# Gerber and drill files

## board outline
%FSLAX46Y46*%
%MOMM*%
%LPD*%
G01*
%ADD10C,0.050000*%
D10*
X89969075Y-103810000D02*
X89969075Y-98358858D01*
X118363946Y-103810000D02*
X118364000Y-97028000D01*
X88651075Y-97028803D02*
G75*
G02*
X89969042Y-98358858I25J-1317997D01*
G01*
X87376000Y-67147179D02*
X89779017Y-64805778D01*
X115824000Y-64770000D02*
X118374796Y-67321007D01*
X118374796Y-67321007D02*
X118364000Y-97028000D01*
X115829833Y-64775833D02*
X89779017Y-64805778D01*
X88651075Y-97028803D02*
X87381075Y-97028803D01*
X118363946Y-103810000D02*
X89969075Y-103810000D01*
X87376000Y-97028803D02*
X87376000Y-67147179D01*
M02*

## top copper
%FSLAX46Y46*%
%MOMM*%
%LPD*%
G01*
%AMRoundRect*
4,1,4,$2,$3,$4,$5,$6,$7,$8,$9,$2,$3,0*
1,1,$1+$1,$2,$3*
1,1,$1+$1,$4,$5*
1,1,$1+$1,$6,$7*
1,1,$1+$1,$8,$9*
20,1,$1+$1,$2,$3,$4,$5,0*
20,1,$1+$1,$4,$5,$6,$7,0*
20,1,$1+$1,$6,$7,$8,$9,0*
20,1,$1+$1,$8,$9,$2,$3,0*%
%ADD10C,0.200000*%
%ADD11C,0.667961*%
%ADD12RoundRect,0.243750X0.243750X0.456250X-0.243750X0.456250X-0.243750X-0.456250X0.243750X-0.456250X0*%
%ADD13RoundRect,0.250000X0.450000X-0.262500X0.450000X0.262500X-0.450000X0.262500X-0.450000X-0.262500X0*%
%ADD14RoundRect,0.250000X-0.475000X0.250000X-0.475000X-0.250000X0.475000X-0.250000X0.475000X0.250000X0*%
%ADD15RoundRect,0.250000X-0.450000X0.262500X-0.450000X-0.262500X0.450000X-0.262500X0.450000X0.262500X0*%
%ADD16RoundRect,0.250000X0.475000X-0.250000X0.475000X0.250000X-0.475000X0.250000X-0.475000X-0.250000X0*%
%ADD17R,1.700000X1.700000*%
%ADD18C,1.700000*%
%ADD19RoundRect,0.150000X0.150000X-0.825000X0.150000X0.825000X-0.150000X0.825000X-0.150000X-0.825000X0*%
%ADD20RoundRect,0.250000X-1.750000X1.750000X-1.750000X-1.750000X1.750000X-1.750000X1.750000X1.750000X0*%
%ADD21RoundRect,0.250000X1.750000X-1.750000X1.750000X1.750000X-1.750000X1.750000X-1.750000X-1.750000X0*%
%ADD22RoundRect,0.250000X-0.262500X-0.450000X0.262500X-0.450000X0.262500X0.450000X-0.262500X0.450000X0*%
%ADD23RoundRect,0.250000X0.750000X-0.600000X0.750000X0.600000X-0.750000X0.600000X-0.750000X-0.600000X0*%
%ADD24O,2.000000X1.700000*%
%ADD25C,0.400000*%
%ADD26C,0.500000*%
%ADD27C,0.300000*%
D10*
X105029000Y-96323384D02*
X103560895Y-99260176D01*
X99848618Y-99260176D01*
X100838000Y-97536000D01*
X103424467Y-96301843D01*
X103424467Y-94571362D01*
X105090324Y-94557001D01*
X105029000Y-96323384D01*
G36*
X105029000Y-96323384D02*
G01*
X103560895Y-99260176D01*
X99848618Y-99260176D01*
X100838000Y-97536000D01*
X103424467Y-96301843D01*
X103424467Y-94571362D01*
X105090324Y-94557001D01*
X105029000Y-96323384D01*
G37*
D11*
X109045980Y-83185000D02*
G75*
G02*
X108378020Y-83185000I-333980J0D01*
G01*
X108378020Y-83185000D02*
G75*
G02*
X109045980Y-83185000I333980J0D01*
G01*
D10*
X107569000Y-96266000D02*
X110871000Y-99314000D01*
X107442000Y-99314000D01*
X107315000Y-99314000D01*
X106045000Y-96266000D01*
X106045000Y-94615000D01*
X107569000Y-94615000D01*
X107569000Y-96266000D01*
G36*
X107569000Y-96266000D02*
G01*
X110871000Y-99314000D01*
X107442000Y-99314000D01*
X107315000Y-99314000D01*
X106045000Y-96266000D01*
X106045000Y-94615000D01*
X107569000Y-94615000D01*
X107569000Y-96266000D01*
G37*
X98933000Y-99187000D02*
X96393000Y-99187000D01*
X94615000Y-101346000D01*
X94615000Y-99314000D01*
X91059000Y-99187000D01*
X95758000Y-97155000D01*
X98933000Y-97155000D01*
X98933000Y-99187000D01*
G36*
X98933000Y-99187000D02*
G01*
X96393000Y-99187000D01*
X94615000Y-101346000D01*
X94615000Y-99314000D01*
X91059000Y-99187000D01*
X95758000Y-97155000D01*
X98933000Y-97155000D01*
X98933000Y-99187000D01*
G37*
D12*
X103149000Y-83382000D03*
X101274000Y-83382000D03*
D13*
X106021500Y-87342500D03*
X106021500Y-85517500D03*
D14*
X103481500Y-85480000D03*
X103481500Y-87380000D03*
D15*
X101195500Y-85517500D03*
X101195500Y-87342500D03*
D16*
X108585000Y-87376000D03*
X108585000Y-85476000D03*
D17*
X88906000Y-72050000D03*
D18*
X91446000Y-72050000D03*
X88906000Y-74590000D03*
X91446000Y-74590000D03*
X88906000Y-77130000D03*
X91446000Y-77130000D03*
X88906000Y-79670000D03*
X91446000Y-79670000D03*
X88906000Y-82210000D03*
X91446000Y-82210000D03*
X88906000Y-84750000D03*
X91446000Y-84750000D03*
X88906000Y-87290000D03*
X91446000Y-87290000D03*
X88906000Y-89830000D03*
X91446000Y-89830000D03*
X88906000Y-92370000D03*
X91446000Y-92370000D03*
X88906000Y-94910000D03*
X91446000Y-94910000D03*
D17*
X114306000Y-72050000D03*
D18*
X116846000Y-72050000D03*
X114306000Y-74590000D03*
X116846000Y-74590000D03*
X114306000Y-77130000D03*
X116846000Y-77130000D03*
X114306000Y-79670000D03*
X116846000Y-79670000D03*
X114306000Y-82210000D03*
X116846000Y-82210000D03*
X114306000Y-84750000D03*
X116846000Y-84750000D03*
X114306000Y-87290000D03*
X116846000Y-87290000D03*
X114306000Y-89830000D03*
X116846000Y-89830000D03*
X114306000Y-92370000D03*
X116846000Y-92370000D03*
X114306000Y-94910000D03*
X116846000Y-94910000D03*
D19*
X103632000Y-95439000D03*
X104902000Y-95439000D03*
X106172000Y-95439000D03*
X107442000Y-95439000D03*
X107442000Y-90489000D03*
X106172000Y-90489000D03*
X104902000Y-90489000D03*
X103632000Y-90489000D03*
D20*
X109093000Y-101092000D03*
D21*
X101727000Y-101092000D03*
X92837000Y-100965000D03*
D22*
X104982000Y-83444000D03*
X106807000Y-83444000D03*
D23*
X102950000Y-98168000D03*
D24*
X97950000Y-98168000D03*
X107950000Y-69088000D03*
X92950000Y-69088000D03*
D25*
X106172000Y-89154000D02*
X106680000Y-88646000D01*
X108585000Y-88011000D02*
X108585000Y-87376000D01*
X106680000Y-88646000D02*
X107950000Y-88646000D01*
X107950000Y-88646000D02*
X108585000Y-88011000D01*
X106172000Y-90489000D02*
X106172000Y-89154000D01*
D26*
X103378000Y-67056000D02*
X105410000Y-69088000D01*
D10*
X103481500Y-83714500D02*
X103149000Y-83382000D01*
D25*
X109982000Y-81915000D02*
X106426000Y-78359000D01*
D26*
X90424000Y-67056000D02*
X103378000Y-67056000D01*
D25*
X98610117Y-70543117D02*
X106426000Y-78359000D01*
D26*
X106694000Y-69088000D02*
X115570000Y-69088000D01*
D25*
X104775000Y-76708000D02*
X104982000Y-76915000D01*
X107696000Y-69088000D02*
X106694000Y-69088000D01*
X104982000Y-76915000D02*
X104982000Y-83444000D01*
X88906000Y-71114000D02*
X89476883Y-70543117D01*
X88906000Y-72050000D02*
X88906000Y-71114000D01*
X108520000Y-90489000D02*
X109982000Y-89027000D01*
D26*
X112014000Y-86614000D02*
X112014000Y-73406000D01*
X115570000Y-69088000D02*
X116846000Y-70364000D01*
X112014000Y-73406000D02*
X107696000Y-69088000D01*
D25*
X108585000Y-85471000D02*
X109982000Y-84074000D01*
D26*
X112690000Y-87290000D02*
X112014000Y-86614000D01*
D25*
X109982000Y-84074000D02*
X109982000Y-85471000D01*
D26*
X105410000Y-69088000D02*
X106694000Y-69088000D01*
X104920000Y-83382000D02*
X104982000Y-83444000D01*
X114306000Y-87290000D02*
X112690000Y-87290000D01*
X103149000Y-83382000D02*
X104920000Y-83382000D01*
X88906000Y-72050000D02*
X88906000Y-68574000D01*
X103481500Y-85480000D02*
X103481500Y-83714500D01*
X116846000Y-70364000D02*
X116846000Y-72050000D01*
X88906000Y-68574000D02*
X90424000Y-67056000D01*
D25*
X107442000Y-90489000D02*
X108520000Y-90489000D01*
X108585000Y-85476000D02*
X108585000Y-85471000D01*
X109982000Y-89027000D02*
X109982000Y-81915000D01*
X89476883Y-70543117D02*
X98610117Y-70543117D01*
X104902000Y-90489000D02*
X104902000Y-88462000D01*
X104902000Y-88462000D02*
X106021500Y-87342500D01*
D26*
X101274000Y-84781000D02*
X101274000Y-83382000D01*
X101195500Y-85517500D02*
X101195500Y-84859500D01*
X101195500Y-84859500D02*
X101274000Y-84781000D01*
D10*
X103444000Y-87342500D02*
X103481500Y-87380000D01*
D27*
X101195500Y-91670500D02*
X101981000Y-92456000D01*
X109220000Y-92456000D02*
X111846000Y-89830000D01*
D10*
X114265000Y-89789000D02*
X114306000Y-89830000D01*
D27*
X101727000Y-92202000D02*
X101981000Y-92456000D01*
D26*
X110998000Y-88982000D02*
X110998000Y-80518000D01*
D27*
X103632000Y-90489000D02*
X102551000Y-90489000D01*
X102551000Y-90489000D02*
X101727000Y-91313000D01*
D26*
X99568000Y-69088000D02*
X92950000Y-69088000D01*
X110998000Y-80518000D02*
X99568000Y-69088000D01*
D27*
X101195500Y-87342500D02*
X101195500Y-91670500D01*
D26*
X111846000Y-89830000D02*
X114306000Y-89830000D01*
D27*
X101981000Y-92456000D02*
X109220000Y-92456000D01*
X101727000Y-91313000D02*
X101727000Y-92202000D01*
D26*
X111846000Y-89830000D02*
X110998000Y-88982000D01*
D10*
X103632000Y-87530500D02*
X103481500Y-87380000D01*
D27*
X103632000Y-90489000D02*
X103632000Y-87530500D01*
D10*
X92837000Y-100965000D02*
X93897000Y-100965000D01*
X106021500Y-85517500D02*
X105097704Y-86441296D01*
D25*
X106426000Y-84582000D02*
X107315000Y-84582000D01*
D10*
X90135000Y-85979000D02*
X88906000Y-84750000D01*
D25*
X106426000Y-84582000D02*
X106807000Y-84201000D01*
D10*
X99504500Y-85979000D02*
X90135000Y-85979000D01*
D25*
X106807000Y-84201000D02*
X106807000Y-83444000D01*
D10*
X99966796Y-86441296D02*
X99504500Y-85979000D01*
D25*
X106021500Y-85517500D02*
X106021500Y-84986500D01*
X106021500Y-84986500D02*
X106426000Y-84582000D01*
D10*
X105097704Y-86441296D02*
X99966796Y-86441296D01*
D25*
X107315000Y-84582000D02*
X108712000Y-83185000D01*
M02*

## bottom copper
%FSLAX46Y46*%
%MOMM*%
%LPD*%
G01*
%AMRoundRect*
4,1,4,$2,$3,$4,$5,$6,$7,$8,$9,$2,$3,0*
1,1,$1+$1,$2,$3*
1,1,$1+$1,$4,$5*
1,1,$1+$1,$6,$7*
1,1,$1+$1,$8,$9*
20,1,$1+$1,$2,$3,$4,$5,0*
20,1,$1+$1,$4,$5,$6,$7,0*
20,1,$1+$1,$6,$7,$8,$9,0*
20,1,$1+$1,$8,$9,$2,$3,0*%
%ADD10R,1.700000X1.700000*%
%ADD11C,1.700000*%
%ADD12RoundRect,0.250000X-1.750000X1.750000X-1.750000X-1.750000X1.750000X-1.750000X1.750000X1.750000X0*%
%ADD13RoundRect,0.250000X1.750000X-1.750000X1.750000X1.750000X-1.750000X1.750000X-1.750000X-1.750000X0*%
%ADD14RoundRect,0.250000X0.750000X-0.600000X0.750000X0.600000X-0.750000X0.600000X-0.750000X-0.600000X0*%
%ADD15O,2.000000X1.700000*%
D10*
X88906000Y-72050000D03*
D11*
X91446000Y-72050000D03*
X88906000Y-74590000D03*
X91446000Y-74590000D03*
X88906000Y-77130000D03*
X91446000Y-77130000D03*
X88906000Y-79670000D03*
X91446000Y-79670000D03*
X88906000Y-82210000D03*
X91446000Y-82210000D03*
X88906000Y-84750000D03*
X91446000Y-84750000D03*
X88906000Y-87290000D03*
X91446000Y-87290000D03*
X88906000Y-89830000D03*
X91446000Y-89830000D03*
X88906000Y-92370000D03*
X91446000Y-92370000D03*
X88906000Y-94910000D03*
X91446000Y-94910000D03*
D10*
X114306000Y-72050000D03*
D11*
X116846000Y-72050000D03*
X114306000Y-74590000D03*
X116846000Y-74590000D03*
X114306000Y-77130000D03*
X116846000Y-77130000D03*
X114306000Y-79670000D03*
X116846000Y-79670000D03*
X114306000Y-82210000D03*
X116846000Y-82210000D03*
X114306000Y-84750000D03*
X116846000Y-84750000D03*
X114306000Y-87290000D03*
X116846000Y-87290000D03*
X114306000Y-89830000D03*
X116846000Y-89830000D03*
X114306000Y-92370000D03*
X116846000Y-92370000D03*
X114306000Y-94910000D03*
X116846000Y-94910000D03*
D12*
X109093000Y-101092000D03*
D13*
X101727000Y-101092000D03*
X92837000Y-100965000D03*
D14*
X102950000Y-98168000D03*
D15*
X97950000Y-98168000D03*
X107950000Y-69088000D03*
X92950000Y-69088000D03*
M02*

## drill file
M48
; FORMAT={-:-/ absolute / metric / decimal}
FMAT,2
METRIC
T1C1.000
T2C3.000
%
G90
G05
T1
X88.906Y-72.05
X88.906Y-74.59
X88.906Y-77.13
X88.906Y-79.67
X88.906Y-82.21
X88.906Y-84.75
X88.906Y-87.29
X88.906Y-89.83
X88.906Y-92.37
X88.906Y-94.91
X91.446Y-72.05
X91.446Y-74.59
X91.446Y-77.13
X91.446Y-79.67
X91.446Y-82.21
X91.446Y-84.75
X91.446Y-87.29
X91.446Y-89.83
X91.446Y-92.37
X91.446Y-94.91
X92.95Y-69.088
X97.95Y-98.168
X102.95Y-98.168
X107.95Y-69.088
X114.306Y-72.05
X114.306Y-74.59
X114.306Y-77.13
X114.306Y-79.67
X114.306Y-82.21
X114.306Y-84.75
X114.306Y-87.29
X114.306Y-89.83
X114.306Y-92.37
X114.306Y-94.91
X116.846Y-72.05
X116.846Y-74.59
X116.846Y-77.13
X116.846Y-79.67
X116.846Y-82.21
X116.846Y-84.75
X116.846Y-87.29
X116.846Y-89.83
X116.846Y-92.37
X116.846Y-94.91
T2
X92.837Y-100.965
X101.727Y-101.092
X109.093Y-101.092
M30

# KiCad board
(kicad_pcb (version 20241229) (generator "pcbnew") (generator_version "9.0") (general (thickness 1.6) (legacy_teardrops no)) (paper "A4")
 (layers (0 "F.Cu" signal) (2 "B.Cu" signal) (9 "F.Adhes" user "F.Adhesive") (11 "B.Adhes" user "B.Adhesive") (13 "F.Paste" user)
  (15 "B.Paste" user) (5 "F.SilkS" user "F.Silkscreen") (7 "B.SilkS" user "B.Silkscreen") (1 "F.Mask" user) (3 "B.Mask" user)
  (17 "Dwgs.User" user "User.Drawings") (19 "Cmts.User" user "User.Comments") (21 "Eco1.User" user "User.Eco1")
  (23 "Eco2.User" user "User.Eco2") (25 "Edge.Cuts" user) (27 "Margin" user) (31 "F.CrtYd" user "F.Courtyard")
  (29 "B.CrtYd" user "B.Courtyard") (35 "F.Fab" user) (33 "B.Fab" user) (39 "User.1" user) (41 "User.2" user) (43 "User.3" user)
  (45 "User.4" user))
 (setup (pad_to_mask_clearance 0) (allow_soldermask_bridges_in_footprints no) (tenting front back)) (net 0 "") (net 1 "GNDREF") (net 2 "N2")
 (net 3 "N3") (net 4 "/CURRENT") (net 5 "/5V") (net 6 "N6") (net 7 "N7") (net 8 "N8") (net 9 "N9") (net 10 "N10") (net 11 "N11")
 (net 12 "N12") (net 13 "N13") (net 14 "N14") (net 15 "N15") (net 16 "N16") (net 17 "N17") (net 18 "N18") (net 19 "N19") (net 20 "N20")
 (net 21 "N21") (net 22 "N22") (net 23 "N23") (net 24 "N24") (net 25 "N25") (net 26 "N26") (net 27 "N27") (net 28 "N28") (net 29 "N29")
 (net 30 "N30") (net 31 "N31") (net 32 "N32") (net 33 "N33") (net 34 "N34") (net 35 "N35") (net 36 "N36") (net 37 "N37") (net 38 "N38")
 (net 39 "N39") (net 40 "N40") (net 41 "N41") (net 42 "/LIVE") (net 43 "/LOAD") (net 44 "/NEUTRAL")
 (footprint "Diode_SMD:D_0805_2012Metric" (layer "F.Cu") (at 102.2115 83.382 180)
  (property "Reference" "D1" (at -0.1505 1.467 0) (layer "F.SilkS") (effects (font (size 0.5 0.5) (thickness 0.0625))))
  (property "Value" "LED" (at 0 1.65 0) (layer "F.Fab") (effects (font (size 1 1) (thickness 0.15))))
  (pad "1" smd roundrect (at -0.9375 0 180) (size 0.975 1.4) (layers "F.Cu" "F.Mask" "F.Paste") (roundrect_rratio 0.25) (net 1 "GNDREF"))
  (pad "2" smd roundrect (at 0.9375 0 180) (size 0.975 1.4) (layers "F.Cu" "F.Mask" "F.Paste") (roundrect_rratio 0.25) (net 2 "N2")))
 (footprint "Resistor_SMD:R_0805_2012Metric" (layer "F.Cu") (at 106.0215 86.43 90)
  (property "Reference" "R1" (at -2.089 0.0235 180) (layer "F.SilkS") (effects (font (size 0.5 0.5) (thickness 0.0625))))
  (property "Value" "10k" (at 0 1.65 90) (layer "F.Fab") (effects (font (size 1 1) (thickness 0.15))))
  (pad "1" smd roundrect (at -0.9125 0 90) (size 1.025 1.4) (layers "F.Cu" "F.Mask" "F.Paste") (roundrect_rratio 0.243902) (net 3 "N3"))
  (pad "2" smd roundrect (at 0.9125 0 90) (size 1.025 1.4) (layers "F.Cu" "F.Mask" "F.Paste") (roundrect_rratio 0.243902) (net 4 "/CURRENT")))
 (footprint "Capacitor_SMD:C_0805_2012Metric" (layer "F.Cu") (at 103.4815 86.43 -90)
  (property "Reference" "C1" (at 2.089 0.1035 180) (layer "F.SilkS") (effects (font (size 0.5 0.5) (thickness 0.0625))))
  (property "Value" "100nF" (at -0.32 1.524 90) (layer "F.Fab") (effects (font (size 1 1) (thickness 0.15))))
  (pad "1" smd roundrect (at -0.95 0 270) (size 1 1.45) (layers "F.Cu" "F.Mask" "F.Paste") (roundrect_rratio 0.25) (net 1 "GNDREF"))
  (pad "2" smd roundrect (at 0.95 0 270) (size 1 1.45) (layers "F.Cu" "F.Mask" "F.Paste") (roundrect_rratio 0.25) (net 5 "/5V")))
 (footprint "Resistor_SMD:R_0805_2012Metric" (layer "F.Cu") (at 101.1955 86.43 -90)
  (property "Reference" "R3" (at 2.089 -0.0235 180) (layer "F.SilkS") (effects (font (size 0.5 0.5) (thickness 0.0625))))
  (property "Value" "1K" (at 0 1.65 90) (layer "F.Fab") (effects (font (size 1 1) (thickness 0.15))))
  (pad "1" smd roundrect (at -0.9125 0 270) (size 1.025 1.4) (layers "F.Cu" "F.Mask" "F.Paste") (roundrect_rratio 0.243902) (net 2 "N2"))
  (pad "2" smd roundrect (at 0.9125 0 270) (size 1.025 1.4) (layers "F.Cu" "F.Mask" "F.Paste") (roundrect_rratio 0.243902) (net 5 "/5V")))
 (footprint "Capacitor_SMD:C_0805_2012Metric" (layer "F.Cu") (at 108.585 86.426 90)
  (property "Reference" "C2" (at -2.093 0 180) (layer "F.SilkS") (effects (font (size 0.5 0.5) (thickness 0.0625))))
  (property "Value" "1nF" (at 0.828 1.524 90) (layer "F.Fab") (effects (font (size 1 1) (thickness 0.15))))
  (pad "1" smd roundrect (at -0.95 0 90) (size 1 1.45) (layers "F.Cu" "F.Mask" "F.Paste") (roundrect_rratio 0.25) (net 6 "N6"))
  (pad "2" smd roundrect (at 0.95 0 90) (size 1 1.45) (layers "F.Cu" "F.Mask" "F.Paste") (roundrect_rratio 0.25) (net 1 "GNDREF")))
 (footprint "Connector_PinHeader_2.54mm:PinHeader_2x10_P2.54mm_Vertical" (layer "F.Cu") (at 88.906 72.05)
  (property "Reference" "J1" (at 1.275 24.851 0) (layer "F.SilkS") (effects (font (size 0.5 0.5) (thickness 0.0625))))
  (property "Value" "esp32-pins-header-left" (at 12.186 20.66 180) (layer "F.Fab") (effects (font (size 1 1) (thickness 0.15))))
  (pad "1" thru_hole rect (at 0 0) (size 1.7 1.7) (drill 1) (layers "*.Cu" "*.Mask") (remove_unused_layers no) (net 1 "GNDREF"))
  (pad "2" thru_hole circle (at 2.54 0) (size 1.7 1.7) (drill 1) (layers "*.Cu" "*.Mask") (remove_unused_layers no) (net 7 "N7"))
  (pad "3" thru_hole circle (at 0 2.54) (size 1.7 1.7) (drill 1) (layers "*.Cu" "*.Mask") (remove_unused_layers no) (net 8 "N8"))
  (pad "4" thru_hole circle (at 2.54 2.54) (size 1.7 1.7) (drill 1) (layers "*.Cu" "*.Mask") (remove_unused_layers no) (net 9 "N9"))
  (pad "5" thru_hole circle (at 0 5.08) (size 1.7 1.7) (drill 1) (layers "*.Cu" "*.Mask") (remove_unused_layers no) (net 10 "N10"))
  (pad "6" thru_hole circle (at 2.54 5.08) (size 1.7 1.7) (drill 1) (layers "*.Cu" "*.Mask") (remove_unused_layers no) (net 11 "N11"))
  (pad "7" thru_hole circle (at 0 7.62) (size 1.7 1.7) (drill 1) (layers "*.Cu" "*.Mask") (remove_unused_layers no) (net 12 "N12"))
  (pad "8" thru_hole circle (at 2.54 7.62) (size 1.7 1.7) (drill 1) (layers "*.Cu" "*.Mask") (remove_unused_layers no) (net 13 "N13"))
  (pad "9" thru_hole circle (at 0 10.16) (size 1.7 1.7) (drill 1) (layers "*.Cu" "*.Mask") (remove_unused_layers no) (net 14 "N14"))
  (pad "10" thru_hole circle (at 2.54 10.16) (size 1.7 1.7) (drill 1) (layers "*.Cu" "*.Mask") (remove_unused_layers no) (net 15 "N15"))
  (pad "11" thru_hole circle (at 0 12.7) (size 1.7 1.7) (drill 1) (layers "*.Cu" "*.Mask") (remove_unused_layers no) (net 4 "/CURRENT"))
  (pad "12" thru_hole circle (at 2.54 12.7) (size 1.7 1.7) (drill 1) (layers "*.Cu" "*.Mask") (remove_unused_layers no) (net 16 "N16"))
  (pad "13" thru_hole circle (at 0 15.24) (size 1.7 1.7) (drill 1) (layers "*.Cu" "*.Mask") (remove_unused_layers no) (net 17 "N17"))
  (pad "14" thru_hole circle (at 2.54 15.24) (size 1.7 1.7) (drill 1) (layers "*.Cu" "*.Mask") (remove_unused_layers no) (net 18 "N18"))
  (pad "15" thru_hole circle (at 0 17.78) (size 1.7 1.7) (drill 1) (layers "*.Cu" "*.Mask") (remove_unused_layers no) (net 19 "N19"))
  (pad "16" thru_hole circle (at 2.54 17.78) (size 1.7 1.7) (drill 1) (layers "*.Cu" "*.Mask") (remove_unused_layers no) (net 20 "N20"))
  (pad "17" thru_hole circle (at 0 20.32) (size 1.7 1.7) (drill 1) (layers "*.Cu" "*.Mask") (remove_unused_layers no) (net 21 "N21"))
  (pad "18" thru_hole circle (at 2.54 20.32) (size 1.7 1.7) (drill 1) (layers "*.Cu" "*.Mask") (remove_unused_layers no) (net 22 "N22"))
  (pad "19" thru_hole circle (at 0 22.86) (size 1.7 1.7) (drill 1) (layers "*.Cu" "*.Mask") (remove_unused_layers no) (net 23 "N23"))
  (pad "20" thru_hole circle (at 2.54 22.86) (size 1.7 1.7) (drill 1) (layers "*.Cu" "*.Mask") (remove_unused_layers no) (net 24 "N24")))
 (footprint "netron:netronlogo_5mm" (layer "F.Cu") (at 95.25 74.041)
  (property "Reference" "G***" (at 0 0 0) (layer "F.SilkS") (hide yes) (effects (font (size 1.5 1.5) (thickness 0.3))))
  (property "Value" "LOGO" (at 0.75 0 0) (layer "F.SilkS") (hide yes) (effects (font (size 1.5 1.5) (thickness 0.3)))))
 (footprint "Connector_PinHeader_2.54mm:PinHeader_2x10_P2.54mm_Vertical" (layer "F.Cu") (at 114.306 72.05)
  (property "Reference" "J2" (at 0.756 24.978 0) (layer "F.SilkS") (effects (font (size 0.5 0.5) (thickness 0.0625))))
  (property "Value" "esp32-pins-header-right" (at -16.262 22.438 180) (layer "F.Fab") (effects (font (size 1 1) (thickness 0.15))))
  (pad "1" thru_hole rect (at 0 0) (size 1.7 1.7) (drill 1) (layers "*.Cu" "*.Mask") (remove_unused_layers no) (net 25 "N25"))
  (pad "2" thru_hole circle (at 2.54 0) (size 1.7 1.7) (drill 1) (layers "*.Cu" "*.Mask") (remove_unused_layers no) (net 1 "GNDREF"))
  (pad "3" thru_hole circle (at 0 2.54) (size 1.7 1.7) (drill 1) (layers "*.Cu" "*.Mask") (remove_unused_layers no) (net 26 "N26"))
  (pad "4" thru_hole circle (at 2.54 2.54) (size 1.7 1.7) (drill 1) (layers "*.Cu" "*.Mask") (remove_unused_layers no) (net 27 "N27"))
  (pad "5" thru_hole circle (at 0 5.08) (size 1.7 1.7) (drill 1) (layers "*.Cu" "*.Mask") (remove_unused_layers no) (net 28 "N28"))
  (pad "6" thru_hole circle (at 2.54 5.08) (size 1.7 1.7) (drill 1) (layers "*.Cu" "*.Mask") (remove_unused_layers no) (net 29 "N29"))
  (pad "7" thru_hole circle (at 0 7.62) (size 1.7 1.7) (drill 1) (layers "*.Cu" "*.Mask") (remove_unused_layers no) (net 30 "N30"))
  (pad "8" thru_hole circle (at 2.54 7.62) (size 1.7 1.7) (drill 1) (layers "*.Cu" "*.Mask") (remove_unused_layers no) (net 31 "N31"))
  (pad "9" thru_hole circle (at 0 10.16) (size 1.7 1.7) (drill 1) (layers "*.Cu" "*.Mask") (remove_unused_layers no) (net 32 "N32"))
  (pad "10" thru_hole circle (at 2.54 10.16) (size 1.7 1.7) (drill 1) (layers "*.Cu" "*.Mask") (remove_unused_layers no) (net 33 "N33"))
  (pad "11" thru_hole circle (at 0 12.7) (size 1.7 1.7) (drill 1) (layers "*.Cu" "*.Mask") (remove_unused_layers no) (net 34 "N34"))
  (pad "12" thru_hole circle (at 2.54 12.7) (size 1.7 1.7) (drill 1) (layers "*.Cu" "*.Mask") (remove_unused_layers no) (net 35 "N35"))
  (pad "13" thru_hole circle (at 0 15.24) (size 1.7 1.7) (drill 1) (layers "*.Cu" "*.Mask") (remove_unused_layers no) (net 1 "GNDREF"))
  (pad "14" thru_hole circle (at 2.54 15.24) (size 1.7 1.7) (drill 1) (layers "*.Cu" "*.Mask") (remove_unused_layers no) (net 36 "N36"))
  (pad "15" thru_hole circle (at 0 17.78) (size 1.7 1.7) (drill 1) (layers "*.Cu" "*.Mask") (remove_unused_layers no) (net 5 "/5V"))
  (pad "16" thru_hole circle (at 2.54 17.78) (size 1.7 1.7) (drill 1) (layers "*.Cu" "*.Mask") (remove_unused_layers no) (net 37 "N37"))
  (pad "17" thru_hole circle (at 0 20.32) (size 1.7 1.7) (drill 1) (layers "*.Cu" "*.Mask") (remove_unused_layers no) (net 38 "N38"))
  (pad "18" thru_hole circle (at 2.54 20.32) (size 1.7 1.7) (drill 1) (layers "*.Cu" "*.Mask") (remove_unused_layers no) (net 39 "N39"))
  (pad "19" thru_hole circle (at 0 22.86) (size 1.7 1.7) (drill 1) (layers "*.Cu" "*.Mask") (remove_unused_layers no) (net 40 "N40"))
  (pad "20" thru_hole circle (at 2.54 22.86) (size 1.7 1.7) (drill 1) (layers "*.Cu" "*.Mask") (remove_unused_layers no) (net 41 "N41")))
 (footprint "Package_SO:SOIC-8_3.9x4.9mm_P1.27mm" (layer "F.Cu") (at 105.537 92.964 90)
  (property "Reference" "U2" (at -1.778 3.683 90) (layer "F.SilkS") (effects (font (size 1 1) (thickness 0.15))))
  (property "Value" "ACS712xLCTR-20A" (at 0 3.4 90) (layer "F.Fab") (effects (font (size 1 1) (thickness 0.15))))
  (pad "1" smd roundrect (at -2.475 -1.905 90) (size 1.95 0.6) (layers "F.Cu" "F.Mask" "F.Paste") (roundrect_rratio 0.25) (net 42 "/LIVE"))
  (pad "2" smd roundrect (at -2.475 -0.635 90) (size 1.95 0.6) (layers "F.Cu" "F.Mask" "F.Paste") (roundrect_rratio 0.25) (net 42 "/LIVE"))
  (pad "3" smd roundrect (at -2.475 0.635 90) (size 1.95 0.6) (layers "F.Cu" "F.Mask" "F.Paste") (roundrect_rratio 0.25) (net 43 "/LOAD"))
  (pad "4" smd roundrect (at -2.475 1.905 90) (size 1.95 0.6) (layers "F.Cu" "F.Mask" "F.Paste") (roundrect_rratio 0.25) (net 43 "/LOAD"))
  (pad "5" smd roundrect (at 2.475 1.905 90) (size 1.95 0.6) (layers "F.Cu" "F.Mask" "F.Paste") (roundrect_rratio 0.25) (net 1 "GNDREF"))
  (pad "6" smd roundrect (at 2.475 0.635 90) (size 1.95 0.6) (layers "F.Cu" "F.Mask" "F.Paste") (roundrect_rratio 0.25) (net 6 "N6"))
  (pad "7" smd roundrect (at 2.475 -0.635 90) (size 1.95 0.6) (layers "F.Cu" "F.Mask" "F.Paste") (roundrect_rratio 0.25) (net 3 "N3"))
  (pad "8" smd roundrect (at 2.475 -1.905 90) (size 1.95 0.6) (layers "F.Cu" "F.Mask" "F.Paste") (roundrect_rratio 0.25) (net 5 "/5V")))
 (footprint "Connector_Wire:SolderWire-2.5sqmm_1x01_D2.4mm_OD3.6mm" (layer "F.Cu") (at 109.093 101.092 -90)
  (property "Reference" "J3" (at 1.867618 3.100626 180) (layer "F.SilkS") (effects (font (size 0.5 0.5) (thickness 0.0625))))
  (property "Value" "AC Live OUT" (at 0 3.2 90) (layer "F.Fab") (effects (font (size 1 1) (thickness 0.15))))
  (pad "1" thru_hole roundrect (at 0 0 270) (size 4 4) (drill 3) (layers "*.Cu" "*.Mask") (remove_unused_layers no)
   (roundrect_rratio 0.0625) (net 43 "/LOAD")))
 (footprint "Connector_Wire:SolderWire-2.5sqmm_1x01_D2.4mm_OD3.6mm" (layer "F.Cu") (at 101.727 101.092 90)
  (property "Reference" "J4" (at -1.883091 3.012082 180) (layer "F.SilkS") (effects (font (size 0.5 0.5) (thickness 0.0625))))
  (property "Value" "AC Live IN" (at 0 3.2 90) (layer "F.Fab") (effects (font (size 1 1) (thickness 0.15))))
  (pad "1" thru_hole roundrect (at 0 0 90) (size 4 4) (drill 3) (layers "*.Cu" "*.Mask") (remove_unused_layers no) (roundrect_rratio 0.0625)
   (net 42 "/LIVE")))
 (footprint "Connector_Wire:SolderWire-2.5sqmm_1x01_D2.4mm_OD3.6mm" (layer "F.Cu") (at 92.837 100.965 90)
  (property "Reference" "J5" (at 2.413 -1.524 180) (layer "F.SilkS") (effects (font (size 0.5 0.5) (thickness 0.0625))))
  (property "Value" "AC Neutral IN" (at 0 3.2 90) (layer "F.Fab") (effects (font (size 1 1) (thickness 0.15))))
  (pad "1" thru_hole roundrect (at 0 0 90) (size 4 4) (drill 3) (layers "*.Cu" "*.Mask") (remove_unused_layers no) (roundrect_rratio 0.0625)
   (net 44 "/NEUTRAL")))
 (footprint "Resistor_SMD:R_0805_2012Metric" (layer "F.Cu") (at 105.8945 83.444)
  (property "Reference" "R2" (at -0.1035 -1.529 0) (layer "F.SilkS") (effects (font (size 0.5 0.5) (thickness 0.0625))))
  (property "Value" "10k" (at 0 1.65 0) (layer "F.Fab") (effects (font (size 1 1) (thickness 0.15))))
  (pad "1" smd roundrect (at -0.9125 0) (size 1.025 1.4) (layers "F.Cu" "F.Mask" "F.Paste") (roundrect_rratio 0.243902) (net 1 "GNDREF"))
  (pad "2" smd roundrect (at 0.9125 0) (size 1.025 1.4) (layers "F.Cu" "F.Mask" "F.Paste") (roundrect_rratio 0.243902) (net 4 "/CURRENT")))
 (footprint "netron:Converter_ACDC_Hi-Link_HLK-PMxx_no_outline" (layer "B.Cu") (at 102.95 98.168 90)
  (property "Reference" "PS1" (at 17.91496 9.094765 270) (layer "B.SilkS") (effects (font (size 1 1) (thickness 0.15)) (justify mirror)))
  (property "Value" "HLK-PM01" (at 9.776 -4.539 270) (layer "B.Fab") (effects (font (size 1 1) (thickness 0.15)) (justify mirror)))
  (pad "1" thru_hole roundrect (at 0 0 90) (size 1.7 2) (drill 1) (layers "*.Cu" "*.Mask") (remove_unused_layers no)
   (roundrect_rratio 0.147059) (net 42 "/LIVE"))
  (pad "2" thru_hole oval (at 0 -5 90) (size 1.7 2) (drill 1) (layers "*.Cu" "*.Mask") (remove_unused_layers no) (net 44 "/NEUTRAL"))
  (pad "3" thru_hole oval (at 29.08 5 90) (size 1.7 2) (drill 1) (layers "*.Cu" "*.Mask") (remove_unused_layers no) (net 1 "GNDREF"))
  (pad "4" thru_hole oval (at 29.08 -10 90) (size 1.7 2) (drill 1) (layers "*.Cu" "*.Mask") (remove_unused_layers no) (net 5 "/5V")))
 (gr_poly
  (pts (xy 100.838 97.536) (xy 103.424467 96.301843) (xy 103.424467 94.571362) (xy 105.090324 94.557001) (xy 105.029 96.323384)
   (xy 103.560895 99.260176) (xy 99.848618 99.260176))
  (stroke (width 0.2) (type solid)) (fill yes) (layer "F.Cu") (net 42))
 (gr_circle (center 108.712 83.185) (end 109.22 83.439) (stroke (width 0.2) (type solid)) (fill yes) (layer "F.Cu") (net 4))
 (gr_poly
  (pts (xy 107.569 94.615) (xy 106.045 94.615) (xy 106.045 96.266) (xy 107.315 99.314) (xy 107.442 99.314) (xy 110.871 99.314)
   (xy 107.569 96.266))
  (stroke (width 0.2) (type solid)) (fill yes) (layer "F.Cu") (net 43))
 (gr_poly
  (pts (xy 91.059 99.187) (xy 95.758 97.155) (xy 98.933 97.155) (xy 98.933 99.187) (xy 96.393 99.187) (xy 94.615 101.346) (xy 94.615 99.314))
  (stroke (width 0.2) (type solid)) (fill yes) (layer "F.Cu") (net 44))
 (gr_line (start 89.969075 103.81) (end 89.969075 98.358858) (stroke (width 0.05) (type default)) (layer "Edge.Cuts"))
 (gr_line (start 118.363946 103.81) (end 118.364 97.028) (stroke (width 0.05) (type default)) (layer "Edge.Cuts"))
 (gr_arc (start 88.651075 97.028803) (mid 89.58733 97.419102) (end 89.969075 98.358858) (stroke (width 0.05) (type default))
  (layer "Edge.Cuts"))
 (gr_line (start 87.376 67.147179) (end 89.779017 64.805778) (stroke (width 0.05) (type default)) (layer "Edge.Cuts"))
 (gr_line (start 115.824 64.77) (end 118.374796 67.321007) (stroke (width 0.05) (type default)) (layer "Edge.Cuts"))
 (gr_line (start 118.374796 67.321007) (end 118.364 97.028) (stroke (width 0.05) (type default)) (layer "Edge.Cuts"))
 (gr_line (start 115.829833 64.775833) (end 89.779017 64.805778) (stroke (width 0.05) (type default)) (layer "Edge.Cuts"))
 (gr_line (start 88.651075 97.028803) (end 87.381075 97.028803) (stroke (width 0.05) (type default)) (layer "Edge.Cuts"))
 (gr_line (start 118.363946 103.81) (end 89.969075 103.81) (stroke (width 0.05) (type default)) (layer "Edge.Cuts"))
 (gr_line (start 87.376 97.028803) (end 87.376 67.147179) (stroke (width 0.05) (type default)) (layer "Edge.Cuts"))
 (segment (start 106.172 89.154) (end 106.68 88.646) (width 0.4) (layer "F.Cu") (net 6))
 (segment (start 108.585 88.011) (end 108.585 87.376) (width 0.4) (layer "F.Cu") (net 6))
 (segment (start 106.68 88.646) (end 107.95 88.646) (width 0.4) (layer "F.Cu") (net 6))
 (segment (start 107.95 88.646) (end 108.585 88.011) (width 0.4) (layer "F.Cu") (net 6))
 (segment (start 106.172 90.489) (end 106.172 89.154) (width 0.4) (layer "F.Cu") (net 6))
 (segment (start 103.378 67.056) (end 105.41 69.088) (width 0.5) (layer "F.Cu") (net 1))
 (segment (start 103.4815 83.7145) (end 103.149 83.382) (width 0.2) (layer "F.Cu") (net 1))
 (segment (start 109.982 81.915) (end 106.426 78.359) (width 0.4) (layer "F.Cu") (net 1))
 (segment (start 90.424 67.056) (end 103.378 67.056) (width 0.5) (layer "F.Cu") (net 1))
 (segment (start 98.610117 70.543117) (end 106.426 78.359) (width 0.4) (layer "F.Cu") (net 1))
 (segment (start 106.694 69.088) (end 115.57 69.088) (width 0.5) (layer "F.Cu") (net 1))
 (segment (start 104.775 76.708) (end 104.982 76.915) (width 0.4) (layer "F.Cu") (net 1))
 (segment (start 107.696 69.088) (end 106.694 69.088) (width 0.4) (layer "F.Cu") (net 1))
 (segment (start 104.982 76.915) (end 104.982 83.444) (width 0.4) (layer "F.Cu") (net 1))
 (segment (start 88.906 71.114) (end 89.476883 70.543117) (width 0.4) (layer "F.Cu") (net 1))
 (segment (start 88.906 72.05) (end 88.906 71.114) (width 0.4) (layer "F.Cu") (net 1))
 (segment (start 108.52 90.489) (end 109.982 89.027) (width 0.4) (layer "F.Cu") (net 1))
 (segment (start 112.014 86.614) (end 112.014 73.406) (width 0.5) (layer "F.Cu") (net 1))
 (segment (start 115.57 69.088) (end 116.846 70.364) (width 0.5) (layer "F.Cu") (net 1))
 (segment (start 112.014 73.406) (end 107.696 69.088) (width 0.5) (layer "F.Cu") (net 1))
 (segment (start 108.585 85.471) (end 109.982 84.074) (width 0.4) (layer "F.Cu") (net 1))
 (segment (start 112.69 87.29) (end 112.014 86.614) (width 0.5) (layer "F.Cu") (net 1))
 (segment (start 109.982 84.074) (end 109.982 85.471) (width 0.4) (layer "F.Cu") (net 1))
 (segment (start 105.41 69.088) (end 106.694 69.088) (width 0.5) (layer "F.Cu") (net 1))
 (segment (start 104.92 83.382) (end 104.982 83.444) (width 0.5) (layer "F.Cu") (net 1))
 (segment (start 114.306 87.29) (end 112.69 87.29) (width 0.5) (layer "F.Cu") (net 1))
 (segment (start 103.149 83.382) (end 104.92 83.382) (width 0.5) (layer "F.Cu") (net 1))
 (segment (start 88.906 72.05) (end 88.906 68.574) (width 0.5) (layer "F.Cu") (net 1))
 (segment (start 103.4815 85.48) (end 103.4815 83.7145) (width 0.5) (layer "F.Cu") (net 1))
 (segment (start 116.846 70.364) (end 116.846 72.05) (width 0.5) (layer "F.Cu") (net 1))
 (segment (start 88.906 68.574) (end 90.424 67.056) (width 0.5) (layer "F.Cu") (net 1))
 (segment (start 107.442 90.489) (end 108.52 90.489) (width 0.4) (layer "F.Cu") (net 1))
 (segment (start 108.585 85.476) (end 108.585 85.471) (width 0.4) (layer "F.Cu") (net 1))
 (segment (start 109.982 89.027) (end 109.982 81.915) (width 0.4) (layer "F.Cu") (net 1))
 (segment (start 89.476883 70.543117) (end 98.610117 70.543117) (width 0.4) (layer "F.Cu") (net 1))
 (segment (start 104.902 90.489) (end 104.902 88.462) (width 0.4) (layer "F.Cu") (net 3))
 (segment (start 104.902 88.462) (end 106.0215 87.3425) (width 0.4) (layer "F.Cu") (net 3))
 (segment (start 101.274 84.781) (end 101.274 83.382) (width 0.5) (layer "F.Cu") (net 2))
 (segment (start 101.1955 85.5175) (end 101.1955 84.8595) (width 0.5) (layer "F.Cu") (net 2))
 (segment (start 101.1955 84.8595) (end 101.274 84.781) (width 0.5) (layer "F.Cu") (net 2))
 (segment (start 103.444 87.3425) (end 103.4815 87.38) (width 0.2) (layer "F.Cu") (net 5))
 (segment (start 101.1955 91.6705) (end 101.981 92.456) (width 0.3) (layer "F.Cu") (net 5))
 (segment (start 109.22 92.456) (end 111.846 89.83) (width 0.3) (layer "F.Cu") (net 5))
 (segment (start 114.265 89.789) (end 114.306 89.83) (width 0.2) (layer "F.Cu") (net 5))
 (segment (start 101.727 92.202) (end 101.981 92.456) (width 0.3) (layer "F.Cu") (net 5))
 (segment (start 110.998 88.982) (end 110.998 80.518) (width 0.5) (layer "F.Cu") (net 5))
 (segment (start 103.632 90.489) (end 102.551 90.489) (width 0.3) (layer "F.Cu") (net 5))
 (segment (start 102.551 90.489) (end 101.727 91.313) (width 0.3) (layer "F.Cu") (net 5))
 (segment (start 99.568 69.088) (end 92.95 69.088) (width 0.5) (layer "F.Cu") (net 5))
 (segment (start 110.998 80.518) (end 99.568 69.088) (width 0.5) (layer "F.Cu") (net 5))
 (segment (start 101.1955 87.3425) (end 101.1955 91.6705) (width 0.3) (layer "F.Cu") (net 5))
 (segment (start 111.846 89.83) (end 114.306 89.83) (width 0.5) (layer "F.Cu") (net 5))
 (segment (start 101.981 92.456) (end 109.22 92.456) (width 0.3) (layer "F.Cu") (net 5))
 (segment (start 101.727 91.313) (end 101.727 92.202) (width 0.3) (layer "F.Cu") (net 5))
 (segment (start 111.846 89.83) (end 110.998 88.982) (width 0.5) (layer "F.Cu") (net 5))
 (segment (start 103.632 87.5305) (end 103.4815 87.38) (width 0.2) (layer "F.Cu") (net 5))
 (segment (start 103.632 90.489) (end 103.632 87.5305) (width 0.3) (layer "F.Cu") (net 5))
 (segment (start 92.837 100.965) (end 93.897 100.965) (width 0.2) (layer "F.Cu") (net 44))
 (segment (start 106.0215 85.5175) (end 105.097704 86.441296) (width 0.2) (layer "F.Cu") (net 4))
 (segment (start 106.426 84.582) (end 107.315 84.582) (width 0.4) (layer "F.Cu") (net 4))
 (segment (start 90.135 85.979) (end 88.906 84.75) (width 0.2) (layer "F.Cu") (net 4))
 (segment (start 106.426 84.582) (end 106.807 84.201) (width 0.4) (layer "F.Cu") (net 4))
 (segment (start 99.5045 85.979) (end 90.135 85.979) (width 0.2) (layer "F.Cu") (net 4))
 (segment (start 106.807 84.201) (end 106.807 83.444) (width 0.4) (layer "F.Cu") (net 4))
 (segment (start 99.966796 86.441296) (end 99.5045 85.979) (width 0.2) (layer "F.Cu") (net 4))
 (segment (start 106.0215 85.5175) (end 106.0215 84.9865) (width 0.4) (layer "F.Cu") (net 4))
 (segment (start 106.0215 84.9865) (end 106.426 84.582) (width 0.4) (layer "F.Cu") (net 4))
 (segment (start 105.097704 86.441296) (end 99.966796 86.441296) (width 0.2) (layer "F.Cu") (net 4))
 (segment (start 107.315 84.582) (end 108.712 83.185) (width 0.4) (layer "F.Cu") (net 4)))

